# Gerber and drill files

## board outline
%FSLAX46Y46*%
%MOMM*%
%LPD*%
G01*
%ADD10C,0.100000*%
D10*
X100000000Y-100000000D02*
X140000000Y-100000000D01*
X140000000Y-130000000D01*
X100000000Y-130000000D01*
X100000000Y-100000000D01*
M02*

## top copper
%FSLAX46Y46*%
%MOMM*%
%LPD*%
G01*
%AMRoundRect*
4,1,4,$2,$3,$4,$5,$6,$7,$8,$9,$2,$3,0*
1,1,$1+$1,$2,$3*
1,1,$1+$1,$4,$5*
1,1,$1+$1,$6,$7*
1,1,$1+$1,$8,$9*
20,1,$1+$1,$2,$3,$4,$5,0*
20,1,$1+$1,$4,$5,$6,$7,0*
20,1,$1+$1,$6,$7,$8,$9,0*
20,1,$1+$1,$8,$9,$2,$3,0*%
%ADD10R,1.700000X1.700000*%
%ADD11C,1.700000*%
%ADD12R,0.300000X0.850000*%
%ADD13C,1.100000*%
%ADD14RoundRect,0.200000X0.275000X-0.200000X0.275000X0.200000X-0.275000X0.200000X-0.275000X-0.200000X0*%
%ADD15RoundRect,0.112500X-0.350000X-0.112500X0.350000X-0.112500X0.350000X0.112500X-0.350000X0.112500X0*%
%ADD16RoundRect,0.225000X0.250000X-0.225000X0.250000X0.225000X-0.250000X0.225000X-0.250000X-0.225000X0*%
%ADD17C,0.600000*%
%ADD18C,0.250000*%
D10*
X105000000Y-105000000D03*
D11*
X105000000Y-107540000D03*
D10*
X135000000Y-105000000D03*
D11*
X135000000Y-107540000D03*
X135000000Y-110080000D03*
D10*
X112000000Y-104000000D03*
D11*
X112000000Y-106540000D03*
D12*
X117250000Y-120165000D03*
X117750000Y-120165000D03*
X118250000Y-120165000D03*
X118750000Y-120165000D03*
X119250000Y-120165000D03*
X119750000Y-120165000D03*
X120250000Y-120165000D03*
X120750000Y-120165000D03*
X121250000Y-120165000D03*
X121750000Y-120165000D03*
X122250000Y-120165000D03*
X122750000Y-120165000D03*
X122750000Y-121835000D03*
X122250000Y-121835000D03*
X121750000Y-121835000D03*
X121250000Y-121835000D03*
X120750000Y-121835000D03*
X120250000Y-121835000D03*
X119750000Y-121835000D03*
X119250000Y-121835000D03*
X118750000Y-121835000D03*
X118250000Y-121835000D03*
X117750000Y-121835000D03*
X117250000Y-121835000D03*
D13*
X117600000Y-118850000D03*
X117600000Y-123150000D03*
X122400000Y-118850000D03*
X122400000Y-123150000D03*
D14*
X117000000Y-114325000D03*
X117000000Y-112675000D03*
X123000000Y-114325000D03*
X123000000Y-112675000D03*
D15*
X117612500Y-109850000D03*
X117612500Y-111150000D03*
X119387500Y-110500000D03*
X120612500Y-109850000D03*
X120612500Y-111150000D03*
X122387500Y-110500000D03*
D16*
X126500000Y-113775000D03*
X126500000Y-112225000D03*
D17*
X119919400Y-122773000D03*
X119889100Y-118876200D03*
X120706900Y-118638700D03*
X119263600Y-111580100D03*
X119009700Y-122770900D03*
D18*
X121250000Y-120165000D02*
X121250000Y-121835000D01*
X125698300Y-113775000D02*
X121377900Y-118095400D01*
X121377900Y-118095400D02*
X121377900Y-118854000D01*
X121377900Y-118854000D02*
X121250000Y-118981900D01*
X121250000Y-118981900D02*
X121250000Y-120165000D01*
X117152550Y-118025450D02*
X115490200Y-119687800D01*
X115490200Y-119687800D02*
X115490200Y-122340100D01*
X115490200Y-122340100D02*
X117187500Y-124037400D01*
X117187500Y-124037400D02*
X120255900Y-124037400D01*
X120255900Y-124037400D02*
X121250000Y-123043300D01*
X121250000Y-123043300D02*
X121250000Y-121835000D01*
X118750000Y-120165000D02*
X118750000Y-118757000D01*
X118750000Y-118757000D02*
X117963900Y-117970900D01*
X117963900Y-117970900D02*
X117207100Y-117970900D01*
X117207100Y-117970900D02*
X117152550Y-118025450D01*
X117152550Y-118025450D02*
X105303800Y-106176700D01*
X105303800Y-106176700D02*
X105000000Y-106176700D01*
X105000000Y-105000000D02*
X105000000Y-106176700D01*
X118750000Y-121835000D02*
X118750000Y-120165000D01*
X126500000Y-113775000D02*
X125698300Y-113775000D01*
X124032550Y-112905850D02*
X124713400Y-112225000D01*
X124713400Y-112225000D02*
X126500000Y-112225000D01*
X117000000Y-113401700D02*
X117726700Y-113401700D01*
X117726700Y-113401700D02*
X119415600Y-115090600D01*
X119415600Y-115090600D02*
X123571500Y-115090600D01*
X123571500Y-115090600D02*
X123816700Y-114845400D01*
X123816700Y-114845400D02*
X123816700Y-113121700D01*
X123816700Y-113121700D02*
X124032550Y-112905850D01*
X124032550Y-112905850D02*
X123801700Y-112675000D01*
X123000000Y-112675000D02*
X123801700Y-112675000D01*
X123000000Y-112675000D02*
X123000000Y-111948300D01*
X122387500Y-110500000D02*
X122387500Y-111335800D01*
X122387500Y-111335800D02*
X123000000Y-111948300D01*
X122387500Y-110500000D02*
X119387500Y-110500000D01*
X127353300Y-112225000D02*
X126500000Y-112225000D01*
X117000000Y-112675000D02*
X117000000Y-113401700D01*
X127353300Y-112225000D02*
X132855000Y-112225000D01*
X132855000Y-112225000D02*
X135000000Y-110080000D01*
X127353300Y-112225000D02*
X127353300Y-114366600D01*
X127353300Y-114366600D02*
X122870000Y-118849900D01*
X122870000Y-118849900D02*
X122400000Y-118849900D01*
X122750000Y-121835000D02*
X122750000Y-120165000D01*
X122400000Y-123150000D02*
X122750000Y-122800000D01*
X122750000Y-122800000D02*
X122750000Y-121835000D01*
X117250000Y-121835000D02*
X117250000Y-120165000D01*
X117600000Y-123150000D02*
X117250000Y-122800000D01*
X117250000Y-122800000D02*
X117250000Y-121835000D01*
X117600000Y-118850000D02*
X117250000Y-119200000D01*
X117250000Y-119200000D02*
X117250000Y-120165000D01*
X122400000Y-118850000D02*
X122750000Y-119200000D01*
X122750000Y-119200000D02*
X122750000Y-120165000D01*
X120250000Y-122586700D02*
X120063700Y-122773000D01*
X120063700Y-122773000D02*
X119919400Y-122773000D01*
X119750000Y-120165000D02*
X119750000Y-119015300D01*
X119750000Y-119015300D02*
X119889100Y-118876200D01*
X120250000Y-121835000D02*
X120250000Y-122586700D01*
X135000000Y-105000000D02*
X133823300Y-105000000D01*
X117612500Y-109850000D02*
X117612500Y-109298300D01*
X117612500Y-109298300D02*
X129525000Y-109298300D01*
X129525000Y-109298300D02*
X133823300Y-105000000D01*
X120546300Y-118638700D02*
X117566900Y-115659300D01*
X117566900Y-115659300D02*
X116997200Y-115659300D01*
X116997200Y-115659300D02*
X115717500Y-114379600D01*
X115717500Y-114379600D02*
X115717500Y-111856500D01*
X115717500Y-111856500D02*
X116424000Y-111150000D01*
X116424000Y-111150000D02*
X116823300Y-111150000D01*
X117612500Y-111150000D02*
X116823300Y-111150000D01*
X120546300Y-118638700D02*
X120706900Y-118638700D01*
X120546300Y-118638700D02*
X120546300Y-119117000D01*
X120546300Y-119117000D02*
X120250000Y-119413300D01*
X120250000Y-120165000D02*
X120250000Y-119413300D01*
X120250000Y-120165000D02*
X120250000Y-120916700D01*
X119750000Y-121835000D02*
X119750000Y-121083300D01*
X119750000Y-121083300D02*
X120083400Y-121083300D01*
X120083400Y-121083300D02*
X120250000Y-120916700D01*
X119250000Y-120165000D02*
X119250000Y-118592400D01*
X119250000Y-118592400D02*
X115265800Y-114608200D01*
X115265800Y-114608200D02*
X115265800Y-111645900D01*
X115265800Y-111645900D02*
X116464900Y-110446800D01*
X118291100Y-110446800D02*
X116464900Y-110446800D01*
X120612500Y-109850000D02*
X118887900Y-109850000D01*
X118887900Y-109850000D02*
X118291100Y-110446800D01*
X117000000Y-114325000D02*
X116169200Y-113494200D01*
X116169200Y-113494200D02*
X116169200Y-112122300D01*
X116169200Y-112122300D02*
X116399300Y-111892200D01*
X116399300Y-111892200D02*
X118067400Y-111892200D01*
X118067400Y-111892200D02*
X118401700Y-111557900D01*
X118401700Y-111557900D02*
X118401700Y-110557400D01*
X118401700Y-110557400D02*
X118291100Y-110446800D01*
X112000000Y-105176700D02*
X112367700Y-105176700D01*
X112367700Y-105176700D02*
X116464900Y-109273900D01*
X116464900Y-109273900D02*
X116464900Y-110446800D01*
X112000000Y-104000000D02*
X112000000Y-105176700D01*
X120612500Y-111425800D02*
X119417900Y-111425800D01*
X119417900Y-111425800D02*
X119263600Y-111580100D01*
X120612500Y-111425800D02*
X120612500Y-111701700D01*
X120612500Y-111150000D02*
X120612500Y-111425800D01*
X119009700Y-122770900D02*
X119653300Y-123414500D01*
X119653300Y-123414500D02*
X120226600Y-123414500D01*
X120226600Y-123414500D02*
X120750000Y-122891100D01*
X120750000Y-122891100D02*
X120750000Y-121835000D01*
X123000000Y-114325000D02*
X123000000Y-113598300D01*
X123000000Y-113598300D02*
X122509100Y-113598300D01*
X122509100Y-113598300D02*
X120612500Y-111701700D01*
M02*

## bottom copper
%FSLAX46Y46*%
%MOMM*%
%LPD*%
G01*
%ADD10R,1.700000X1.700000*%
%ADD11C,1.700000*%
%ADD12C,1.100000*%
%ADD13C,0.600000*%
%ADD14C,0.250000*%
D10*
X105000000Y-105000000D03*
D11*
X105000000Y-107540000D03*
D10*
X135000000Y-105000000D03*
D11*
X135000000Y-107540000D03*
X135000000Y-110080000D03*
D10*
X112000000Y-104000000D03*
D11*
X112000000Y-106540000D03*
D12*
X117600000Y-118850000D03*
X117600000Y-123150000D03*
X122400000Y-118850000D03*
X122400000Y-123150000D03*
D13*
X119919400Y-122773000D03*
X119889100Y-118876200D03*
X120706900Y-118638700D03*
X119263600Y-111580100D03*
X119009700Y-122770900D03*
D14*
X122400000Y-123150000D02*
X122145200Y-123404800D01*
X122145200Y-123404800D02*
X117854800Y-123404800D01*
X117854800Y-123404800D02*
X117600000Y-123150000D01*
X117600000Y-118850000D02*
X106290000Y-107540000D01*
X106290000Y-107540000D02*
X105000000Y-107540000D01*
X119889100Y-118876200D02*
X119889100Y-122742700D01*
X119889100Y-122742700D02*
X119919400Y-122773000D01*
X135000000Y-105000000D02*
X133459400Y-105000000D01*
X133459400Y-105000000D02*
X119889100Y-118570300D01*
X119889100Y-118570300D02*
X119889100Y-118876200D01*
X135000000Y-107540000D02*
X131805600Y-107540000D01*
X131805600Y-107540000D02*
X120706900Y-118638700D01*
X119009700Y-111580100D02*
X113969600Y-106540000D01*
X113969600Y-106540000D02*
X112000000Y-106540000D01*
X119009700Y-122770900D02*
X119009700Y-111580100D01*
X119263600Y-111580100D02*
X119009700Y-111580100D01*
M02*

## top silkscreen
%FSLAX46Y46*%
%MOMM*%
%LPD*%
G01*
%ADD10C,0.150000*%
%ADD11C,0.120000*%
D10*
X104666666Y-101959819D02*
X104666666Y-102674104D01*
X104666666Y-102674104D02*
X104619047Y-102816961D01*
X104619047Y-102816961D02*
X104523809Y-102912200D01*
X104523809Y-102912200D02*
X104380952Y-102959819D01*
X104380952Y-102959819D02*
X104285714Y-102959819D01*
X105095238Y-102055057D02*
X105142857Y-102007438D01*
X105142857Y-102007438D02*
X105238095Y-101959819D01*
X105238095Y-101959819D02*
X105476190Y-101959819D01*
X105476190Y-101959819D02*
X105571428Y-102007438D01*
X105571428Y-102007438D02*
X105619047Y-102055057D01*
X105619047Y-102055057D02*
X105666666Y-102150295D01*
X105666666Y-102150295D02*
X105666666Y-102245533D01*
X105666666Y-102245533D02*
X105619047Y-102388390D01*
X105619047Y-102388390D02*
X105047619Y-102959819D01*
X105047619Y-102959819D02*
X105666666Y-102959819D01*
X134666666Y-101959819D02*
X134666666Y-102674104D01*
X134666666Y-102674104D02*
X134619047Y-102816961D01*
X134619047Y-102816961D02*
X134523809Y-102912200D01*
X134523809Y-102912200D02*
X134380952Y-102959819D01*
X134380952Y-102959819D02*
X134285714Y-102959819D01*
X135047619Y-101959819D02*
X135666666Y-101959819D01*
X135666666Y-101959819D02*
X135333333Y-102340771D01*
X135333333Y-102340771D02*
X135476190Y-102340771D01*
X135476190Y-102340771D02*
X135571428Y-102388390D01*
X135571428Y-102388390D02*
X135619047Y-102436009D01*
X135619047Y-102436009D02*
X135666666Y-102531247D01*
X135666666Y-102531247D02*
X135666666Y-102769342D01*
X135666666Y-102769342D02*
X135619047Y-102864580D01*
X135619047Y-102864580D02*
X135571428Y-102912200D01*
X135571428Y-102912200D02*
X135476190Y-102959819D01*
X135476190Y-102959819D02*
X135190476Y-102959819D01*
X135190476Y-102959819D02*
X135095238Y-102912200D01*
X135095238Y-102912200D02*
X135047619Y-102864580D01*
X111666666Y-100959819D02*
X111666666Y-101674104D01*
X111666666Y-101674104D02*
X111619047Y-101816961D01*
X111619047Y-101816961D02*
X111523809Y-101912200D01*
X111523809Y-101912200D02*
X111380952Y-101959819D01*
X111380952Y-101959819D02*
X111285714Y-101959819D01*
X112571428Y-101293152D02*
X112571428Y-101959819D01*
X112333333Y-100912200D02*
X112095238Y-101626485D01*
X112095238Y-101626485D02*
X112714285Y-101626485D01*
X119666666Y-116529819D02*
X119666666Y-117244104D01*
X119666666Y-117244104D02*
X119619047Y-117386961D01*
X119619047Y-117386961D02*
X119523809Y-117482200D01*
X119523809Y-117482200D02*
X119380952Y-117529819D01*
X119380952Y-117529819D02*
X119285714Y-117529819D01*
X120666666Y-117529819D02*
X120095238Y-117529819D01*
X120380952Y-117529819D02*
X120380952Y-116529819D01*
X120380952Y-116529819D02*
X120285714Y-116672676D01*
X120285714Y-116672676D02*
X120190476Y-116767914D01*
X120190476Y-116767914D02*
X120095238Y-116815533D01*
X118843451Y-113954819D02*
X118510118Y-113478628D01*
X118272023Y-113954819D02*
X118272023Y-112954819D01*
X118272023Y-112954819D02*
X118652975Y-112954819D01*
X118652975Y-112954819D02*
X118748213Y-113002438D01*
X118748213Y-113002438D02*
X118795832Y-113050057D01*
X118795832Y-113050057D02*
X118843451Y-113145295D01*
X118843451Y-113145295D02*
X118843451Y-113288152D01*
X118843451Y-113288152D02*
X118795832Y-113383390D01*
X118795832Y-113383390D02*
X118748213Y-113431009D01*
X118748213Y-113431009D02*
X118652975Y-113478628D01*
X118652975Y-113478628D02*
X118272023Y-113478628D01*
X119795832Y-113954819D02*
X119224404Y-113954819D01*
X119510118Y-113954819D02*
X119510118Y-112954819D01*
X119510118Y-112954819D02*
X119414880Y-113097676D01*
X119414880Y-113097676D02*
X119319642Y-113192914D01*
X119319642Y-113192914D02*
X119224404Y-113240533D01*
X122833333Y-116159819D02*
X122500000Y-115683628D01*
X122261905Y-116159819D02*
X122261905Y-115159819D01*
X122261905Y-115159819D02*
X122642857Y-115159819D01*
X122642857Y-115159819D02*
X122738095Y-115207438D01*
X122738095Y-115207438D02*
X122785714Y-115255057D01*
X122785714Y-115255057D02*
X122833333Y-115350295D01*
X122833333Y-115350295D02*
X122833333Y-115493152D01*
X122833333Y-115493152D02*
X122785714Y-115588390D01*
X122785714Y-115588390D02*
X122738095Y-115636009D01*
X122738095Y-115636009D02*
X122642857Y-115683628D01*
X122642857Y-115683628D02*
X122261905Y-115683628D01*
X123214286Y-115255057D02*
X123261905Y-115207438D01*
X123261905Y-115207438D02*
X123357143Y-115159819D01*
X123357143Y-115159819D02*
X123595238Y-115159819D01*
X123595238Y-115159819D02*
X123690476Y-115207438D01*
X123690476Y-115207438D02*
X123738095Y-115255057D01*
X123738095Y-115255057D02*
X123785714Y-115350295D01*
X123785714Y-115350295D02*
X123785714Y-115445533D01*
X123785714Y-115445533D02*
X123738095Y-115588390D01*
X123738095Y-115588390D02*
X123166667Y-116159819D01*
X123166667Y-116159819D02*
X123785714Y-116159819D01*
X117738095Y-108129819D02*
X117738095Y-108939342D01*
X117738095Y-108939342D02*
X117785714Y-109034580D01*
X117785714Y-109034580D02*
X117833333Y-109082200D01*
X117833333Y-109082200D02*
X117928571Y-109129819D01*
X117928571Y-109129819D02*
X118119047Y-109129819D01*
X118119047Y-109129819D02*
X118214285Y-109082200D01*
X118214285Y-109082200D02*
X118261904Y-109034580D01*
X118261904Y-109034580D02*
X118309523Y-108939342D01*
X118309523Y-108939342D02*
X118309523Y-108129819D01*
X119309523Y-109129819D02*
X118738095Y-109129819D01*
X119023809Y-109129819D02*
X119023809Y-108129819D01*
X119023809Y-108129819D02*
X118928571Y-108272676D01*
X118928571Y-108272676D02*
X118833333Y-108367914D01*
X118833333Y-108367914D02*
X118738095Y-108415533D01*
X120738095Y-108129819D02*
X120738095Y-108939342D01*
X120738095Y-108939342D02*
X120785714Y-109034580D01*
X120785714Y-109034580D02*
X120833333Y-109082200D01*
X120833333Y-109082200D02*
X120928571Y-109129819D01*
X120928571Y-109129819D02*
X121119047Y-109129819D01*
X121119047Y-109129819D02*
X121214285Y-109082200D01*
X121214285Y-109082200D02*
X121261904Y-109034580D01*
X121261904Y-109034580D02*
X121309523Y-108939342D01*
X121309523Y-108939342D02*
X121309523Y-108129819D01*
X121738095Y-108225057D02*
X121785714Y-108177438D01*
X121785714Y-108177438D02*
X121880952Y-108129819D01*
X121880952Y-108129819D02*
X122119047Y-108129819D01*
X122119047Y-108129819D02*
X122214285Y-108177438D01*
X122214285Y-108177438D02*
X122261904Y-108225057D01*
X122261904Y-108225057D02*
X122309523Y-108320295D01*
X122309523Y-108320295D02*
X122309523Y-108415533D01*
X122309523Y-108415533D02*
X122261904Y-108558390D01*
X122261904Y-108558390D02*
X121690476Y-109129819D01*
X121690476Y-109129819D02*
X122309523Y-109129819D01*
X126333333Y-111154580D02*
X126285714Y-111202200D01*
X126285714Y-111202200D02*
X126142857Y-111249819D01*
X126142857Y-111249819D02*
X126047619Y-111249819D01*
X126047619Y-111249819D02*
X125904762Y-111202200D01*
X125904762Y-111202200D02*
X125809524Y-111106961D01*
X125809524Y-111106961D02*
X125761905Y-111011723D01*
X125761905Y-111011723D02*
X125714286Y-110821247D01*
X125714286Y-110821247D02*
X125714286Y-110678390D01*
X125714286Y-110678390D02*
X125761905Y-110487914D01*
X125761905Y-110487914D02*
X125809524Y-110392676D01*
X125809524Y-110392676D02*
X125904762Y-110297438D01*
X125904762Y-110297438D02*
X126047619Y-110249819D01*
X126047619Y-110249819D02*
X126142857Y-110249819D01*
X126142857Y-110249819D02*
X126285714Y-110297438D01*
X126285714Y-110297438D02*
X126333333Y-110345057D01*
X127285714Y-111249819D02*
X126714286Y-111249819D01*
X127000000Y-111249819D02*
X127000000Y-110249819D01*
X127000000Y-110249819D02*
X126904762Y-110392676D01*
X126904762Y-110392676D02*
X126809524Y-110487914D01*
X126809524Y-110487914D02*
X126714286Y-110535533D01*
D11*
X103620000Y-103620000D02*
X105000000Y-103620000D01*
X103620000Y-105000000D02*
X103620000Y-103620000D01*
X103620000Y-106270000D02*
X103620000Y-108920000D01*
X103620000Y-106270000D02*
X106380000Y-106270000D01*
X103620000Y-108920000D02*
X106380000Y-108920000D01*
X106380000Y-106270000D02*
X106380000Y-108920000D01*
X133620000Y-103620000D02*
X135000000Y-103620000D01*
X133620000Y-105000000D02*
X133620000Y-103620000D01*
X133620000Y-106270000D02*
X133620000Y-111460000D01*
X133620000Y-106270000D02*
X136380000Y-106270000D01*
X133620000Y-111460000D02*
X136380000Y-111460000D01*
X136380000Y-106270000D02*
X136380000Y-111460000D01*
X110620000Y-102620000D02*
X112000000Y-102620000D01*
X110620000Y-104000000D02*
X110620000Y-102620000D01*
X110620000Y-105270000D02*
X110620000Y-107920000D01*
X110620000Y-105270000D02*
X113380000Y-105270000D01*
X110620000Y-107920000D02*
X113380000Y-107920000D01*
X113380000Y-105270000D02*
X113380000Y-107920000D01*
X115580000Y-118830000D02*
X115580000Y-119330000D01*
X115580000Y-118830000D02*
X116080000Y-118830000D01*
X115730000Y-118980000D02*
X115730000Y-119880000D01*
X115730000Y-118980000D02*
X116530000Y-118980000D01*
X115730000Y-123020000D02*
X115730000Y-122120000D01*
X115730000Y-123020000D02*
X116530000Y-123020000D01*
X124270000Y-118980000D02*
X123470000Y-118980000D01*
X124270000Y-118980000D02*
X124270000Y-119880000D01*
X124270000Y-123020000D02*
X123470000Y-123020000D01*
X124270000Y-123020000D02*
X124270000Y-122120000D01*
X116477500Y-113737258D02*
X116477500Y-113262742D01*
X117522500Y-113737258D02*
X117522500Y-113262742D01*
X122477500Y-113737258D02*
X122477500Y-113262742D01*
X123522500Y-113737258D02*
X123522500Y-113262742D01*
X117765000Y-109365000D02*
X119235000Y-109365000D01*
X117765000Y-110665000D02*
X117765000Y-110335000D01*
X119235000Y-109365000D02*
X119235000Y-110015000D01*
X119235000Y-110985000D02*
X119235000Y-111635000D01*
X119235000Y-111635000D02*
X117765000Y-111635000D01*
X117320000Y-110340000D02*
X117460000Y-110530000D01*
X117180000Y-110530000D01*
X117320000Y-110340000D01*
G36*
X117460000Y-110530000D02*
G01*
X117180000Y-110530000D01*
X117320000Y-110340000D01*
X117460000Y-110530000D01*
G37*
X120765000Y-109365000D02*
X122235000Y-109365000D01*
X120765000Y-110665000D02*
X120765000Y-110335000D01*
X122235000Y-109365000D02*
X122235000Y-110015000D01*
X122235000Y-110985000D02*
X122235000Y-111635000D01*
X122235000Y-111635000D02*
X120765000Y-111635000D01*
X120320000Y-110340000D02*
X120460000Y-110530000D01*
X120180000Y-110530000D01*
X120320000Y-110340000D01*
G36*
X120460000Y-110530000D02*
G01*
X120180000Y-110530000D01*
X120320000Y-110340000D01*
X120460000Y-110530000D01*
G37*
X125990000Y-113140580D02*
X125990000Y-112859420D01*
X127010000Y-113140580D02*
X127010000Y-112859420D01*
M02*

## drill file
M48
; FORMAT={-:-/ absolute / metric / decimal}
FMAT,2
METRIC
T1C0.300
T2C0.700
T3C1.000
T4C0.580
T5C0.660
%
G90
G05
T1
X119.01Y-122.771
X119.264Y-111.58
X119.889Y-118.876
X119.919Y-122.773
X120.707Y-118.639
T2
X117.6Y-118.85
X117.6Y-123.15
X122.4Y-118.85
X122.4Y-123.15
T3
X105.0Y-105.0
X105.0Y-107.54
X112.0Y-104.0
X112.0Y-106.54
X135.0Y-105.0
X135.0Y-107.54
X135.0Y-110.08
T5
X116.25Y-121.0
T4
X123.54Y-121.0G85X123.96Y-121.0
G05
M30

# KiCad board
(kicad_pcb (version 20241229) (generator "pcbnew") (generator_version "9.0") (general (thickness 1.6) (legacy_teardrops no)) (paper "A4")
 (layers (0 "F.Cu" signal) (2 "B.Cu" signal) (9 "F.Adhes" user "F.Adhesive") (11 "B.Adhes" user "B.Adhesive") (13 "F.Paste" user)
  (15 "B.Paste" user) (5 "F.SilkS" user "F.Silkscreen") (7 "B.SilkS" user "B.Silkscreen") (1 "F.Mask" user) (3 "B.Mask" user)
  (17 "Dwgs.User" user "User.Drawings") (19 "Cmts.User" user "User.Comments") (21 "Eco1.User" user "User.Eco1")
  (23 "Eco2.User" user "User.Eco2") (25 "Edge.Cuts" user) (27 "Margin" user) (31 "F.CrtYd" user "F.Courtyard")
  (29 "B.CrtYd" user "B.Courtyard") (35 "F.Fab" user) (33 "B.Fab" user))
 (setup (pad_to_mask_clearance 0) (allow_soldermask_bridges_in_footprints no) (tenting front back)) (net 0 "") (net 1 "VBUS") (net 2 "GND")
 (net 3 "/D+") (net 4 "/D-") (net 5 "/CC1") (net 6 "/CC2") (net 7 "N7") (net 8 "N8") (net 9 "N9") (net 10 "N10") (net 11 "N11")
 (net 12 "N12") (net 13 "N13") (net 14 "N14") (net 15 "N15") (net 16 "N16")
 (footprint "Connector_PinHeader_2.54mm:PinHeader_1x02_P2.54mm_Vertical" (layer "F.Cu") (at 105 105)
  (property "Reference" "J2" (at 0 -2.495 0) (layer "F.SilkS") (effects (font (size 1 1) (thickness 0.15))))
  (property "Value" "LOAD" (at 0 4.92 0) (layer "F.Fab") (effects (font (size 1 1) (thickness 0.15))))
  (fp_line (start -1.38 -1.38) (end 0 -1.38) (stroke (width 0.12) (type solid)) (layer "F.SilkS"))
  (fp_line (start -1.38 0) (end -1.38 -1.38) (stroke (width 0.12) (type solid)) (layer "F.SilkS"))
  (fp_line (start -1.38 1.27) (end -1.38 3.92) (stroke (width 0.12) (type solid)) (layer "F.SilkS"))
  (fp_line (start -1.38 1.27) (end 1.38 1.27) (stroke (width 0.12) (type solid)) (layer "F.SilkS"))
  (fp_line (start -1.38 3.92) (end 1.38 3.92) (stroke (width 0.12) (type solid)) (layer "F.SilkS"))
  (fp_line (start 1.38 1.27) (end 1.38 3.92) (stroke (width 0.12) (type solid)) (layer "F.SilkS"))
  (pad "1" thru_hole rect (at 0 0) (size 1.7 1.7) (drill 1) (layers "*.Cu" "*.Mask") (remove_unused_layers no) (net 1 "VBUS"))
  (pad "2" thru_hole circle (at 0 2.54) (size 1.7 1.7) (drill 1) (layers "*.Cu" "*.Mask") (remove_unused_layers no) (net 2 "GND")))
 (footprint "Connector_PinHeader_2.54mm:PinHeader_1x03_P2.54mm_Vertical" (layer "F.Cu") (at 135 105)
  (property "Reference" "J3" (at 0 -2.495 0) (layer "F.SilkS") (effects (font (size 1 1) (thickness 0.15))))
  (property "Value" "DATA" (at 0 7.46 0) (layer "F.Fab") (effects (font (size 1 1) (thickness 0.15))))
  (fp_line (start -1.38 -1.38) (end 0 -1.38) (stroke (width 0.12) (type solid)) (layer "F.SilkS"))
  (fp_line (start -1.38 0) (end -1.38 -1.38) (stroke (width 0.12) (type solid)) (layer "F.SilkS"))
  (fp_line (start -1.38 1.27) (end -1.38 6.46) (stroke (width 0.12) (type solid)) (layer "F.SilkS"))
  (fp_line (start -1.38 1.27) (end 1.38 1.27) (stroke (width 0.12) (type solid)) (layer "F.SilkS"))
  (fp_line (start -1.38 6.46) (end 1.38 6.46) (stroke (width 0.12) (type solid)) (layer "F.SilkS"))
  (fp_line (start 1.38 1.27) (end 1.38 6.46) (stroke (width 0.12) (type solid)) (layer "F.SilkS"))
  (pad "1" thru_hole rect (at 0 0) (size 1.7 1.7) (drill 1) (layers "*.Cu" "*.Mask") (remove_unused_layers no) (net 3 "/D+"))
  (pad "2" thru_hole circle (at 0 2.54) (size 1.7 1.7) (drill 1) (layers "*.Cu" "*.Mask") (remove_unused_layers no) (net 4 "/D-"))
  (pad "3" thru_hole circle (at 0 5.08) (size 1.7 1.7) (drill 1) (layers "*.Cu" "*.Mask") (remove_unused_layers no) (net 2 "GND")))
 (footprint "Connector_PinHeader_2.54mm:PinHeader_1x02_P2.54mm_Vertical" (layer "F.Cu") (at 112 104)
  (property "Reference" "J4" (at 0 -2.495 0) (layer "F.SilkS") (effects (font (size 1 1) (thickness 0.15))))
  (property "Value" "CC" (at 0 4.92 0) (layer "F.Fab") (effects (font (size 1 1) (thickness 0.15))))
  (fp_line (start -1.38 -1.38) (end 0 -1.38) (stroke (width 0.12) (type solid)) (layer "F.SilkS"))
  (fp_line (start -1.38 0) (end -1.38 -1.38) (stroke (width 0.12) (type solid)) (layer "F.SilkS"))
  (fp_line (start -1.38 1.27) (end -1.38 3.92) (stroke (width 0.12) (type solid)) (layer "F.SilkS"))
  (fp_line (start -1.38 1.27) (end 1.38 1.27) (stroke (width 0.12) (type solid)) (layer "F.SilkS"))
  (fp_line (start -1.38 3.92) (end 1.38 3.92) (stroke (width 0.12) (type solid)) (layer "F.SilkS"))
  (fp_line (start 1.38 1.27) (end 1.38 3.92) (stroke (width 0.12) (type solid)) (layer "F.SilkS"))
  (pad "1" thru_hole rect (at 0 0) (size 1.7 1.7) (drill 1) (layers "*.Cu" "*.Mask") (remove_unused_layers no) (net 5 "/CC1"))
  (pad "2" thru_hole circle (at 0 2.54) (size 1.7 1.7) (drill 1) (layers "*.Cu" "*.Mask") (remove_unused_layers no) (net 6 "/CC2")))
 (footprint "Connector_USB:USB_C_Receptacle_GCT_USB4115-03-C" (layer "F.Cu") (at 120 121)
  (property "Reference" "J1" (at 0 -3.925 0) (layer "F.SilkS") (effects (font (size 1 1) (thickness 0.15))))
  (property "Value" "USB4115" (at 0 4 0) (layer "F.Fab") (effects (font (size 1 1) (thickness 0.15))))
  (fp_line (start -4.42 -2.17) (end -4.42 -1.67) (stroke (width 0.12) (type solid)) (layer "F.SilkS"))
  (fp_line (start -4.42 -2.17) (end -3.92 -2.17) (stroke (width 0.12) (type solid)) (layer "F.SilkS"))
  (fp_line (start -4.27 -2.02) (end -4.27 -1.12) (stroke (width 0.12) (type solid)) (layer "F.SilkS"))
  (fp_line (start -4.27 -2.02) (end -3.47 -2.02) (stroke (width 0.12) (type solid)) (layer "F.SilkS"))
  (fp_line (start -4.27 2.02) (end -4.27 1.12) (stroke (width 0.12) (type solid)) (layer "F.SilkS"))
  (fp_line (start -4.27 2.02) (end -3.47 2.02) (stroke (width 0.12) (type solid)) (layer "F.SilkS"))
  (fp_line (start 4.27 -2.02) (end 3.47 -2.02) (stroke (width 0.12) (type solid)) (layer "F.SilkS"))
  (fp_line (start 4.27 -2.02) (end 4.27 -1.12) (stroke (width 0.12) (type solid)) (layer "F.SilkS"))
  (fp_line (start 4.27 2.02) (end 3.47 2.02) (stroke (width 0.12) (type solid)) (layer "F.SilkS"))
  (fp_line (start 4.27 2.02) (end 4.27 1.12) (stroke (width 0.12) (type solid)) (layer "F.SilkS"))
  (pad "" np_thru_hole circle (at -3.75 0) (size 0.66 0.66) (drill 0.66) (layers "*.Cu" "*.Mask"))
  (pad "" np_thru_hole oval (at 3.75 0) (size 1 0.58) (drill oval 1 0.58) (layers "*.Cu" "*.Mask"))
  (pad "A1" smd rect (at -2.75 -0.835) (size 0.3 0.85) (layers "F.Cu" "F.Mask" "F.Paste") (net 2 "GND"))
  (pad "A2" smd rect (at -2.25 -0.835) (size 0.3 0.85) (layers "F.Cu" "F.Mask" "F.Paste") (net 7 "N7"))
  (pad "A3" smd rect (at -1.75 -0.835) (size 0.3 0.85) (layers "F.Cu" "F.Mask" "F.Paste") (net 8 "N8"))
  (pad "A4" smd rect (at -1.25 -0.835) (size 0.3 0.85) (layers "F.Cu" "F.Mask" "F.Paste") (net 1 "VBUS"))
  (pad "A5" smd rect (at -0.75 -0.835) (size 0.3 0.85) (layers "F.Cu" "F.Mask" "F.Paste") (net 5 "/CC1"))
  (pad "A6" smd rect (at -0.25 -0.835) (size 0.3 0.85) (layers "F.Cu" "F.Mask" "F.Paste") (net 3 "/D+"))
  (pad "A7" smd rect (at 0.25 -0.835) (size 0.3 0.85) (layers "F.Cu" "F.Mask" "F.Paste") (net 4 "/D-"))
  (pad "A8" smd rect (at 0.75 -0.835) (size 0.3 0.85) (layers "F.Cu" "F.Mask" "F.Paste") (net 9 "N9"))
  (pad "A9" smd rect (at 1.25 -0.835) (size 0.3 0.85) (layers "F.Cu" "F.Mask" "F.Paste") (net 1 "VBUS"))
  (pad "A10" smd rect (at 1.75 -0.835) (size 0.3 0.85) (layers "F.Cu" "F.Mask" "F.Paste") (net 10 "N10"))
  (pad "A11" smd rect (at 2.25 -0.835) (size 0.3 0.85) (layers "F.Cu" "F.Mask" "F.Paste") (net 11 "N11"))
  (pad "A12" smd rect (at 2.75 -0.835) (size 0.3 0.85) (layers "F.Cu" "F.Mask" "F.Paste") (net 2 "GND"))
  (pad "B1" smd rect (at 2.75 0.835) (size 0.3 0.85) (layers "F.Cu" "F.Mask" "F.Paste") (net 2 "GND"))
  (pad "B2" smd rect (at 2.25 0.835) (size 0.3 0.85) (layers "F.Cu" "F.Mask" "F.Paste") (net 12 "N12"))
  (pad "B3" smd rect (at 1.75 0.835) (size 0.3 0.85) (layers "F.Cu" "F.Mask" "F.Paste") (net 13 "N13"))
  (pad "B4" smd rect (at 1.25 0.835) (size 0.3 0.85) (layers "F.Cu" "F.Mask" "F.Paste") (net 1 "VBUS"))
  (pad "B5" smd rect (at 0.75 0.835) (size 0.3 0.85) (layers "F.Cu" "F.Mask" "F.Paste") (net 6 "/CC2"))
  (pad "B6" smd rect (at 0.25 0.835) (size 0.3 0.85) (layers "F.Cu" "F.Mask" "F.Paste") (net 3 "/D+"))
  (pad "B7" smd rect (at -0.25 0.835) (size 0.3 0.85) (layers "F.Cu" "F.Mask" "F.Paste") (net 4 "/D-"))
  (pad "B8" smd rect (at -0.75 0.835) (size 0.3 0.85) (layers "F.Cu" "F.Mask" "F.Paste") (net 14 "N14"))
  (pad "B9" smd rect (at -1.25 0.835) (size 0.3 0.85) (layers "F.Cu" "F.Mask" "F.Paste") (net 1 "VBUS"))
  (pad "B10" smd rect (at -1.75 0.835) (size 0.3 0.85) (layers "F.Cu" "F.Mask" "F.Paste") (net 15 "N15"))
  (pad "B11" smd rect (at -2.25 0.835) (size 0.3 0.85) (layers "F.Cu" "F.Mask" "F.Paste") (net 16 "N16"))
  (pad "B12" smd rect (at -2.75 0.835) (size 0.3 0.85) (layers "F.Cu" "F.Mask" "F.Paste") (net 2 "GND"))
  (pad "SH" thru_hole circle (at -2.4 -2.15) (size 1.1 1.1) (drill 0.7) (layers "*.Cu" "*.Mask" "F.Paste") (remove_unused_layers no)
   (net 2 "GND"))
  (pad "SH" thru_hole circle (at -2.4 2.15) (size 1.1 1.1) (drill 0.7) (layers "*.Cu" "*.Mask" "F.Paste") (remove_unused_layers no)
   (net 2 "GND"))
  (pad "SH" thru_hole circle (at 2.4 -2.15) (size 1.1 1.1) (drill 0.7) (layers "*.Cu" "*.Mask" "F.Paste") (remove_unused_layers no)
   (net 2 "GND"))
  (pad "SH" thru_hole circle (at 2.4 2.15) (size 1.1 1.1) (drill 0.7) (layers "*.Cu" "*.Mask" "F.Paste") (remove_unused_layers no)
   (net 2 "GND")))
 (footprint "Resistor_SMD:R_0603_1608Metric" (layer "F.Cu") (at 117 113.5 90)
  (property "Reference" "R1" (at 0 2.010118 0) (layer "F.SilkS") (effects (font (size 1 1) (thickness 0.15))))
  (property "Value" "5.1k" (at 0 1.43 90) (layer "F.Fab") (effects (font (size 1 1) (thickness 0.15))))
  (fp_line (start -0.237258 -0.5225) (end 0.237258 -0.5225) (stroke (width 0.12) (type solid)) (layer "F.SilkS"))
  (fp_line (start -0.237258 0.5225) (end 0.237258 0.5225) (stroke (width 0.12) (type solid)) (layer "F.SilkS"))
  (pad "1" smd roundrect (at -0.825 0 90) (size 0.8 0.95) (layers "F.Cu" "F.Mask" "F.Paste") (roundrect_rratio 0.25) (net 5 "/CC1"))
  (pad "2" smd roundrect (at 0.825 0 90) (size 0.8 0.95) (layers "F.Cu" "F.Mask" "F.Paste") (roundrect_rratio 0.25) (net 2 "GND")))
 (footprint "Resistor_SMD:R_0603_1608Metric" (layer "F.Cu") (at 123 113.5 90)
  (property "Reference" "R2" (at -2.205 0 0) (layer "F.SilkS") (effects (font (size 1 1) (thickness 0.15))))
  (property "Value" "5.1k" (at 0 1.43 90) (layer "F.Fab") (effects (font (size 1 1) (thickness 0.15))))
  (fp_line (start -0.237258 -0.5225) (end 0.237258 -0.5225) (stroke (width 0.12) (type solid)) (layer "F.SilkS"))
  (fp_line (start -0.237258 0.5225) (end 0.237258 0.5225) (stroke (width 0.12) (type solid)) (layer "F.SilkS"))
  (pad "1" smd roundrect (at -0.825 0 90) (size 0.8 0.95) (layers "F.Cu" "F.Mask" "F.Paste") (roundrect_rratio 0.25) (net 6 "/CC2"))
  (pad "2" smd roundrect (at 0.825 0 90) (size 0.8 0.95) (layers "F.Cu" "F.Mask" "F.Paste") (roundrect_rratio 0.25) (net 2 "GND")))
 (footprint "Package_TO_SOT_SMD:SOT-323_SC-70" (layer "F.Cu") (at 118.5 110.5)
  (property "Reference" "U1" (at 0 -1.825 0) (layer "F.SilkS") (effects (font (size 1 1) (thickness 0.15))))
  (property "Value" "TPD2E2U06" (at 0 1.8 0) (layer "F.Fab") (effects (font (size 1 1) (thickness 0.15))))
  (fp_line (start -0.735 -1.135) (end 0.735 -1.135) (stroke (width 0.12) (type solid)) (layer "F.SilkS"))
  (fp_line (start -0.735 0.165) (end -0.735 -0.165) (stroke (width 0.12) (type solid)) (layer "F.SilkS"))
  (fp_line (start 0.735 -1.135) (end 0.735 -0.485) (stroke (width 0.12) (type solid)) (layer "F.SilkS"))
  (fp_line (start 0.735 0.485) (end 0.735 1.135) (stroke (width 0.12) (type solid)) (layer "F.SilkS"))
  (fp_line (start 0.735 1.135) (end -0.735 1.135) (stroke (width 0.12) (type solid)) (layer "F.SilkS"))
  (fp_poly (pts (xy -1.18 -0.16) (xy -1.04 0.03) (xy -1.32 0.03)) (stroke (width 0.12) (type solid)) (fill yes) (layer "F.SilkS"))
  (pad "1" smd roundrect (at -0.8875 -0.65) (size 0.925 0.45) (layers "F.Cu" "F.Mask" "F.Paste") (roundrect_rratio 0.25) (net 3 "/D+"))
  (pad "2" smd roundrect (at -0.8875 0.65) (size 0.925 0.45) (layers "F.Cu" "F.Mask" "F.Paste") (roundrect_rratio 0.25) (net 4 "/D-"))
  (pad "3" smd roundrect (at 0.8875 0) (size 0.925 0.45) (layers "F.Cu" "F.Mask" "F.Paste") (roundrect_rratio 0.25) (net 2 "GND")))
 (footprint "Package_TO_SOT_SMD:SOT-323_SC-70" (layer "F.Cu") (at 121.5 110.5)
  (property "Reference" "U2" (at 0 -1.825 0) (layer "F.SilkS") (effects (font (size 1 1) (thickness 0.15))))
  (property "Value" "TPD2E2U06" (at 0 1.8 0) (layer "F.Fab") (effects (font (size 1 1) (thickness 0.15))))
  (fp_line (start -0.735 -1.135) (end 0.735 -1.135) (stroke (width 0.12) (type solid)) (layer "F.SilkS"))
  (fp_line (start -0.735 0.165) (end -0.735 -0.165) (stroke (width 0.12) (type solid)) (layer "F.SilkS"))
  (fp_line (start 0.735 -1.135) (end 0.735 -0.485) (stroke (width 0.12) (type solid)) (layer "F.SilkS"))
  (fp_line (start 0.735 0.485) (end 0.735 1.135) (stroke (width 0.12) (type solid)) (layer "F.SilkS"))
  (fp_line (start 0.735 1.135) (end -0.735 1.135) (stroke (width 0.12) (type solid)) (layer "F.SilkS"))
  (fp_poly (pts (xy -1.18 -0.16) (xy -1.04 0.03) (xy -1.32 0.03)) (stroke (width 0.12) (type solid)) (fill yes) (layer "F.SilkS"))
  (pad "1" smd roundrect (at -0.8875 -0.65) (size 0.925 0.45) (layers "F.Cu" "F.Mask" "F.Paste") (roundrect_rratio 0.25) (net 5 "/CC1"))
  (pad "2" smd roundrect (at -0.8875 0.65) (size 0.925 0.45) (layers "F.Cu" "F.Mask" "F.Paste") (roundrect_rratio 0.25) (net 6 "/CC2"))
  (pad "3" smd roundrect (at 0.8875 0) (size 0.925 0.45) (layers "F.Cu" "F.Mask" "F.Paste") (roundrect_rratio 0.25) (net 2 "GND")))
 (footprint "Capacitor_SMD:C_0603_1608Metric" (layer "F.Cu") (at 126.5 113 90)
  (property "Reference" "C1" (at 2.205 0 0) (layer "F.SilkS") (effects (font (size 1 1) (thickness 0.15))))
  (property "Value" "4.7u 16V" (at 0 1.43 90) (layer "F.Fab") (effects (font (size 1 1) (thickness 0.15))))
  (fp_line (start -0.14058 -0.51) (end 0.14058 -0.51) (stroke (width 0.12) (type solid)) (layer "F.SilkS"))
  (fp_line (start -0.14058 0.51) (end 0.14058 0.51) (stroke (width 0.12) (type solid)) (layer "F.SilkS"))
  (pad "1" smd roundrect (at -0.775 0 90) (size 0.9 0.95) (layers "F.Cu" "F.Mask" "F.Paste") (roundrect_rratio 0.25) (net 1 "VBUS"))
  (pad "2" smd roundrect (at 0.775 0 90) (size 0.9 0.95) (layers "F.Cu" "F.Mask" "F.Paste") (roundrect_rratio 0.25) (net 2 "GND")))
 (gr_rect (start 100 100) (end 140 130) (stroke (width 0.1) (type default)) (fill no) (layer "Edge.Cuts"))
 (segment (start 121.25 120.165) (end 121.25 121.835) (width 0.25) (layer "F.Cu") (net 1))
 (segment (start 125.6983 113.775) (end 121.3779 118.0954) (width 0.25) (layer "F.Cu") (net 1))
 (segment (start 121.3779 118.0954) (end 121.3779 118.854) (width 0.25) (layer "F.Cu") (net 1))
 (segment (start 121.3779 118.854) (end 121.25 118.9819) (width 0.25) (layer "F.Cu") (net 1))
 (segment (start 121.25 118.9819) (end 121.25 120.165) (width 0.25) (layer "F.Cu") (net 1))
 (segment (start 117.15255 118.02545) (end 115.4902 119.6878) (width 0.25) (layer "F.Cu") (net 1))
 (segment (start 115.4902 119.6878) (end 115.4902 122.3401) (width 0.25) (layer "F.Cu") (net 1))
 (segment (start 115.4902 122.3401) (end 117.1875 124.0374) (width 0.25) (layer "F.Cu") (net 1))
 (segment (start 117.1875 124.0374) (end 120.2559 124.0374) (width 0.25) (layer "F.Cu") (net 1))
 (segment (start 120.2559 124.0374) (end 121.25 123.0433) (width 0.25) (layer "F.Cu") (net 1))
 (segment (start 121.25 123.0433) (end 121.25 121.835) (width 0.25) (layer "F.Cu") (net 1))
 (segment (start 118.75 120.165) (end 118.75 118.757) (width 0.25) (layer "F.Cu") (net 1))
 (segment (start 118.75 118.757) (end 117.9639 117.9709) (width 0.25) (layer "F.Cu") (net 1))
 (segment (start 117.9639 117.9709) (end 117.2071 117.9709) (width 0.25) (layer "F.Cu") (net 1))
 (segment (start 117.2071 117.9709) (end 117.15255 118.02545) (width 0.25) (layer "F.Cu") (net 1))
 (segment (start 117.15255 118.02545) (end 105.3038 106.1767) (width 0.25) (layer "F.Cu") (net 1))
 (segment (start 105.3038 106.1767) (end 105 106.1767) (width 0.25) (layer "F.Cu") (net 1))
 (segment (start 105 105) (end 105 106.1767) (width 0.25) (layer "F.Cu") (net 1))
 (segment (start 118.75 121.835) (end 118.75 120.165) (width 0.25) (layer "F.Cu") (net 1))
 (segment (start 126.5 113.775) (end 125.6983 113.775) (width 0.25) (layer "F.Cu") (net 1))
 (segment (start 124.03255 112.90585) (end 124.7134 112.225) (width 0.25) (layer "F.Cu") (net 2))
 (segment (start 124.7134 112.225) (end 126.5 112.225) (width 0.25) (layer "F.Cu") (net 2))
 (segment (start 117 113.4017) (end 117.7267 113.4017) (width 0.25) (layer "F.Cu") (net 2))
 (segment (start 117.7267 113.4017) (end 119.4156 115.0906) (width 0.25) (layer "F.Cu") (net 2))
 (segment (start 119.4156 115.0906) (end 123.5715 115.0906) (width 0.25) (layer "F.Cu") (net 2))
 (segment (start 123.5715 115.0906) (end 123.8167 114.8454) (width 0.25) (layer "F.Cu") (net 2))
 (segment (start 123.8167 114.8454) (end 123.8167 113.1217) (width 0.25) (layer "F.Cu") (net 2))
 (segment (start 123.8167 113.1217) (end 124.03255 112.90585) (width 0.25) (layer "F.Cu") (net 2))
 (segment (start 124.03255 112.90585) (end 123.8017 112.675) (width 0.25) (layer "F.Cu") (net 2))
 (segment (start 123 112.675) (end 123.8017 112.675) (width 0.25) (layer "F.Cu") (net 2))
 (segment (start 123 112.675) (end 123 111.9483) (width 0.25) (layer "F.Cu") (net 2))
 (segment (start 122.3875 110.5) (end 122.3875 111.3358) (width 0.25) (layer "F.Cu") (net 2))
 (segment (start 122.3875 111.3358) (end 123 111.9483) (width 0.25) (layer "F.Cu") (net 2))
 (segment (start 122.3875 110.5) (end 119.3875 110.5) (width 0.25) (layer "F.Cu") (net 2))
 (segment (start 127.3533 112.225) (end 126.5 112.225) (width 0.25) (layer "F.Cu") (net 2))
 (segment (start 122.4 123.15) (end 122.1452 123.4048) (width 0.25) (layer "B.Cu") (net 2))
 (segment (start 122.1452 123.4048) (end 117.8548 123.4048) (width 0.25) (layer "B.Cu") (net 2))
 (segment (start 117.8548 123.4048) (end 117.6 123.15) (width 0.25) (layer "B.Cu") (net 2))
 (segment (start 117.6 118.85) (end 106.29 107.54) (width 0.25) (layer "B.Cu") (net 2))
 (segment (start 106.29 107.54) (end 105 107.54) (width 0.25) (layer "B.Cu") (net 2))
 (segment (start 117 112.675) (end 117 113.4017) (width 0.25) (layer "F.Cu") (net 2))
 (segment (start 127.3533 112.225) (end 132.855 112.225) (width 0.25) (layer "F.Cu") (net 2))
 (segment (start 132.855 112.225) (end 135 110.08) (width 0.25) (layer "F.Cu") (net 2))
 (segment (start 127.3533 112.225) (end 127.3533 114.3666) (width 0.25) (layer "F.Cu") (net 2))
 (segment (start 127.3533 114.3666) (end 122.87 118.8499) (width 0.25) (layer "F.Cu") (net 2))
 (segment (start 122.87 118.8499) (end 122.4 118.8499) (width 0.25) (layer "F.Cu") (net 2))
 (segment (start 122.75 121.835) (end 122.75 120.165) (width 0.25) (layer "F.Cu") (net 2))
 (segment (start 122.4 123.15) (end 122.75 122.8) (width 0.25) (layer "F.Cu") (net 2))
 (segment (start 122.75 122.8) (end 122.75 121.835) (width 0.25) (layer "F.Cu") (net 2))
 (segment (start 117.25 121.835) (end 117.25 120.165) (width 0.25) (layer "F.Cu") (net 2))
 (segment (start 117.6 123.15) (end 117.25 122.8) (width 0.25) (layer "F.Cu") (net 2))
 (segment (start 117.25 122.8) (end 117.25 121.835) (width 0.25) (layer "F.Cu") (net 2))
 (segment (start 117.6 118.85) (end 117.25 119.2) (width 0.25) (layer "F.Cu") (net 2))
 (segment (start 117.25 119.2) (end 117.25 120.165) (width 0.25) (layer "F.Cu") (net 2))
 (segment (start 122.4 118.85) (end 122.75 119.2) (width 0.25) (layer "F.Cu") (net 2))
 (segment (start 122.75 119.2) (end 122.75 120.165) (width 0.25) (layer "F.Cu") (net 2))
 (segment (start 120.25 122.5867) (end 120.0637 122.773) (width 0.25) (layer "F.Cu") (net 3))
 (segment (start 120.0637 122.773) (end 119.9194 122.773) (width 0.25) (layer "F.Cu") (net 3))
 (segment (start 119.8891 118.8762) (end 119.8891 122.7427) (width 0.25) (layer "B.Cu") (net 3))
 (segment (start 119.8891 122.7427) (end 119.9194 122.773) (width 0.25) (layer "B.Cu") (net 3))
 (segment (start 135 105) (end 133.4594 105) (width 0.25) (layer "B.Cu") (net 3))
 (segment (start 133.4594 105) (end 119.8891 118.5703) (width 0.25) (layer "B.Cu") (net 3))
 (segment (start 119.8891 118.5703) (end 119.8891 118.8762) (width 0.25) (layer "B.Cu") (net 3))
 (segment (start 119.75 120.165) (end 119.75 119.0153) (width 0.25) (layer "F.Cu") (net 3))
 (segment (start 119.75 119.0153) (end 119.8891 118.8762) (width 0.25) (layer "F.Cu") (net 3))
 (segment (start 120.25 121.835) (end 120.25 122.5867) (width 0.25) (layer "F.Cu") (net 3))
 (segment (start 135 105) (end 133.8233 105) (width 0.25) (layer "F.Cu") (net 3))
 (segment (start 117.6125 109.85) (end 117.6125 109.2983) (width 0.25) (layer "F.Cu") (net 3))
 (segment (start 117.6125 109.2983) (end 129.525 109.2983) (width 0.25) (layer "F.Cu") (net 3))
 (segment (start 129.525 109.2983) (end 133.8233 105) (width 0.25) (layer "F.Cu") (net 3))
 (segment (start 120.5463 118.6387) (end 117.5669 115.6593) (width 0.25) (layer "F.Cu") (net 4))
 (segment (start 117.5669 115.6593) (end 116.9972 115.6593) (width 0.25) (layer "F.Cu") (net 4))
 (segment (start 116.9972 115.6593) (end 115.7175 114.3796) (width 0.25) (layer "F.Cu") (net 4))
 (segment (start 115.7175 114.3796) (end 115.7175 111.8565) (width 0.25) (layer "F.Cu") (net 4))
 (segment (start 115.7175 111.8565) (end 116.424 111.15) (width 0.25) (layer "F.Cu") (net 4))
 (segment (start 116.424 111.15) (end 116.8233 111.15) (width 0.25) (layer "F.Cu") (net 4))
 (segment (start 117.6125 111.15) (end 116.8233 111.15) (width 0.25) (layer "F.Cu") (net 4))
 (segment (start 120.5463 118.6387) (end 120.7069 118.6387) (width 0.25) (layer "F.Cu") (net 4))
 (segment (start 135 107.54) (end 131.8056 107.54) (width 0.25) (layer "B.Cu") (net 4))
 (segment (start 131.8056 107.54) (end 120.7069 118.6387) (width 0.25) (layer "B.Cu") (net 4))
 (segment (start 120.5463 118.6387) (end 120.5463 119.117) (width 0.25) (layer "F.Cu") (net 4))
 (segment (start 120.5463 119.117) (end 120.25 119.4133) (width 0.25) (layer "F.Cu") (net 4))
 (segment (start 120.25 120.165) (end 120.25 119.4133) (width 0.25) (layer "F.Cu") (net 4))
 (segment (start 120.25 120.165) (end 120.25 120.9167) (width 0.25) (layer "F.Cu") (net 4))
 (segment (start 119.75 121.835) (end 119.75 121.0833) (width 0.25) (layer "F.Cu") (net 4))
 (segment (start 119.75 121.0833) (end 120.0834 121.0833) (width 0.25) (layer "F.Cu") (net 4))
 (segment (start 120.0834 121.0833) (end 120.25 120.9167) (width 0.25) (layer "F.Cu") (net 4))
 (segment (start 119.25 120.165) (end 119.25 118.5924) (width 0.25) (layer "F.Cu") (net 5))
 (segment (start 119.25 118.5924) (end 115.2658 114.6082) (width 0.25) (layer "F.Cu") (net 5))
 (segment (start 115.2658 114.6082) (end 115.2658 111.6459) (width 0.25) (layer "F.Cu") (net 5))
 (segment (start 115.2658 111.6459) (end 116.4649 110.4468) (width 0.25) (layer "F.Cu") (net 5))
 (segment (start 118.2911 110.4468) (end 116.4649 110.4468) (width 0.25) (layer "F.Cu") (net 5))
 (segment (start 120.6125 109.85) (end 118.8879 109.85) (width 0.25) (layer "F.Cu") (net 5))
 (segment (start 118.8879 109.85) (end 118.2911 110.4468) (width 0.25) (layer "F.Cu") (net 5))
 (segment (start 117 114.325) (end 116.1692 113.4942) (width 0.25) (layer "F.Cu") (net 5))
 (segment (start 116.1692 113.4942) (end 116.1692 112.1223) (width 0.25) (layer "F.Cu") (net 5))
 (segment (start 116.1692 112.1223) (end 116.3993 111.8922) (width 0.25) (layer "F.Cu") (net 5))
 (segment (start 116.3993 111.8922) (end 118.0674 111.8922) (width 0.25) (layer "F.Cu") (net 5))
 (segment (start 118.0674 111.8922) (end 118.4017 111.5579) (width 0.25) (layer "F.Cu") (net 5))
 (segment (start 118.4017 111.5579) (end 118.4017 110.5574) (width 0.25) (layer "F.Cu") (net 5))
 (segment (start 118.4017 110.5574) (end 118.2911 110.4468) (width 0.25) (layer "F.Cu") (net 5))
 (segment (start 112 105.1767) (end 112.3677 105.1767) (width 0.25) (layer "F.Cu") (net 5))
 (segment (start 112.3677 105.1767) (end 116.4649 109.2739) (width 0.25) (layer "F.Cu") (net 5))
 (segment (start 116.4649 109.2739) (end 116.4649 110.4468) (width 0.25) (layer "F.Cu") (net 5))
 (segment (start 112 104) (end 112 105.1767) (width 0.25) (layer "F.Cu") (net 5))
 (segment (start 119.0097 111.5801) (end 113.9696 106.54) (width 0.25) (layer "B.Cu") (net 6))
 (segment (start 113.9696 106.54) (end 112 106.54) (width 0.25) (layer "B.Cu") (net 6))
 (segment (start 119.0097 122.7709) (end 119.0097 111.5801) (width 0.25) (layer "B.Cu") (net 6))
 (segment (start 119.2636 111.5801) (end 119.0097 111.5801) (width 0.25) (layer "B.Cu") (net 6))
 (segment (start 120.6125 111.4258) (end 119.4179 111.4258) (width 0.25) (layer "F.Cu") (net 6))
 (segment (start 119.4179 111.4258) (end 119.2636 111.5801) (width 0.25) (layer "F.Cu") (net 6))
 (segment (start 120.6125 111.4258) (end 120.6125 111.7017) (width 0.25) (layer "F.Cu") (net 6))
 (segment (start 120.6125 111.15) (end 120.6125 111.4258) (width 0.25) (layer "F.Cu") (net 6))
 (segment (start 119.0097 122.7709) (end 119.6533 123.4145) (width 0.25) (layer "F.Cu") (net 6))
 (segment (start 119.6533 123.4145) (end 120.2266 123.4145) (width 0.25) (layer "F.Cu") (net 6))
 (segment (start 120.2266 123.4145) (end 120.75 122.8911) (width 0.25) (layer "F.Cu") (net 6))
 (segment (start 120.75 122.8911) (end 120.75 121.835) (width 0.25) (layer "F.Cu") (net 6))
 (segment (start 123 114.325) (end 123 113.5983) (width 0.25) (layer "F.Cu") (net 6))
 (segment (start 123 113.5983) (end 122.5091 113.5983) (width 0.25) (layer "F.Cu") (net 6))
 (segment (start 122.5091 113.5983) (end 120.6125 111.7017) (width 0.25) (layer "F.Cu") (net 6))
 (via (at 119.9194 122.773) (size 0.6) (drill 0.3) (layers "F.Cu" "B.Cu") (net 3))
 (via (at 119.8891 118.8762) (size 0.6) (drill 0.3) (layers "F.Cu" "B.Cu") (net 3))
 (via (at 120.7069 118.6387) (size 0.6) (drill 0.3) (layers "F.Cu" "B.Cu") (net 4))
 (via (at 119.2636 111.5801) (size 0.6) (drill 0.3) (layers "F.Cu" "B.Cu") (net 6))
 (via (at 119.0097 122.7709) (size 0.6) (drill 0.3) (layers "F.Cu" "B.Cu") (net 6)))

